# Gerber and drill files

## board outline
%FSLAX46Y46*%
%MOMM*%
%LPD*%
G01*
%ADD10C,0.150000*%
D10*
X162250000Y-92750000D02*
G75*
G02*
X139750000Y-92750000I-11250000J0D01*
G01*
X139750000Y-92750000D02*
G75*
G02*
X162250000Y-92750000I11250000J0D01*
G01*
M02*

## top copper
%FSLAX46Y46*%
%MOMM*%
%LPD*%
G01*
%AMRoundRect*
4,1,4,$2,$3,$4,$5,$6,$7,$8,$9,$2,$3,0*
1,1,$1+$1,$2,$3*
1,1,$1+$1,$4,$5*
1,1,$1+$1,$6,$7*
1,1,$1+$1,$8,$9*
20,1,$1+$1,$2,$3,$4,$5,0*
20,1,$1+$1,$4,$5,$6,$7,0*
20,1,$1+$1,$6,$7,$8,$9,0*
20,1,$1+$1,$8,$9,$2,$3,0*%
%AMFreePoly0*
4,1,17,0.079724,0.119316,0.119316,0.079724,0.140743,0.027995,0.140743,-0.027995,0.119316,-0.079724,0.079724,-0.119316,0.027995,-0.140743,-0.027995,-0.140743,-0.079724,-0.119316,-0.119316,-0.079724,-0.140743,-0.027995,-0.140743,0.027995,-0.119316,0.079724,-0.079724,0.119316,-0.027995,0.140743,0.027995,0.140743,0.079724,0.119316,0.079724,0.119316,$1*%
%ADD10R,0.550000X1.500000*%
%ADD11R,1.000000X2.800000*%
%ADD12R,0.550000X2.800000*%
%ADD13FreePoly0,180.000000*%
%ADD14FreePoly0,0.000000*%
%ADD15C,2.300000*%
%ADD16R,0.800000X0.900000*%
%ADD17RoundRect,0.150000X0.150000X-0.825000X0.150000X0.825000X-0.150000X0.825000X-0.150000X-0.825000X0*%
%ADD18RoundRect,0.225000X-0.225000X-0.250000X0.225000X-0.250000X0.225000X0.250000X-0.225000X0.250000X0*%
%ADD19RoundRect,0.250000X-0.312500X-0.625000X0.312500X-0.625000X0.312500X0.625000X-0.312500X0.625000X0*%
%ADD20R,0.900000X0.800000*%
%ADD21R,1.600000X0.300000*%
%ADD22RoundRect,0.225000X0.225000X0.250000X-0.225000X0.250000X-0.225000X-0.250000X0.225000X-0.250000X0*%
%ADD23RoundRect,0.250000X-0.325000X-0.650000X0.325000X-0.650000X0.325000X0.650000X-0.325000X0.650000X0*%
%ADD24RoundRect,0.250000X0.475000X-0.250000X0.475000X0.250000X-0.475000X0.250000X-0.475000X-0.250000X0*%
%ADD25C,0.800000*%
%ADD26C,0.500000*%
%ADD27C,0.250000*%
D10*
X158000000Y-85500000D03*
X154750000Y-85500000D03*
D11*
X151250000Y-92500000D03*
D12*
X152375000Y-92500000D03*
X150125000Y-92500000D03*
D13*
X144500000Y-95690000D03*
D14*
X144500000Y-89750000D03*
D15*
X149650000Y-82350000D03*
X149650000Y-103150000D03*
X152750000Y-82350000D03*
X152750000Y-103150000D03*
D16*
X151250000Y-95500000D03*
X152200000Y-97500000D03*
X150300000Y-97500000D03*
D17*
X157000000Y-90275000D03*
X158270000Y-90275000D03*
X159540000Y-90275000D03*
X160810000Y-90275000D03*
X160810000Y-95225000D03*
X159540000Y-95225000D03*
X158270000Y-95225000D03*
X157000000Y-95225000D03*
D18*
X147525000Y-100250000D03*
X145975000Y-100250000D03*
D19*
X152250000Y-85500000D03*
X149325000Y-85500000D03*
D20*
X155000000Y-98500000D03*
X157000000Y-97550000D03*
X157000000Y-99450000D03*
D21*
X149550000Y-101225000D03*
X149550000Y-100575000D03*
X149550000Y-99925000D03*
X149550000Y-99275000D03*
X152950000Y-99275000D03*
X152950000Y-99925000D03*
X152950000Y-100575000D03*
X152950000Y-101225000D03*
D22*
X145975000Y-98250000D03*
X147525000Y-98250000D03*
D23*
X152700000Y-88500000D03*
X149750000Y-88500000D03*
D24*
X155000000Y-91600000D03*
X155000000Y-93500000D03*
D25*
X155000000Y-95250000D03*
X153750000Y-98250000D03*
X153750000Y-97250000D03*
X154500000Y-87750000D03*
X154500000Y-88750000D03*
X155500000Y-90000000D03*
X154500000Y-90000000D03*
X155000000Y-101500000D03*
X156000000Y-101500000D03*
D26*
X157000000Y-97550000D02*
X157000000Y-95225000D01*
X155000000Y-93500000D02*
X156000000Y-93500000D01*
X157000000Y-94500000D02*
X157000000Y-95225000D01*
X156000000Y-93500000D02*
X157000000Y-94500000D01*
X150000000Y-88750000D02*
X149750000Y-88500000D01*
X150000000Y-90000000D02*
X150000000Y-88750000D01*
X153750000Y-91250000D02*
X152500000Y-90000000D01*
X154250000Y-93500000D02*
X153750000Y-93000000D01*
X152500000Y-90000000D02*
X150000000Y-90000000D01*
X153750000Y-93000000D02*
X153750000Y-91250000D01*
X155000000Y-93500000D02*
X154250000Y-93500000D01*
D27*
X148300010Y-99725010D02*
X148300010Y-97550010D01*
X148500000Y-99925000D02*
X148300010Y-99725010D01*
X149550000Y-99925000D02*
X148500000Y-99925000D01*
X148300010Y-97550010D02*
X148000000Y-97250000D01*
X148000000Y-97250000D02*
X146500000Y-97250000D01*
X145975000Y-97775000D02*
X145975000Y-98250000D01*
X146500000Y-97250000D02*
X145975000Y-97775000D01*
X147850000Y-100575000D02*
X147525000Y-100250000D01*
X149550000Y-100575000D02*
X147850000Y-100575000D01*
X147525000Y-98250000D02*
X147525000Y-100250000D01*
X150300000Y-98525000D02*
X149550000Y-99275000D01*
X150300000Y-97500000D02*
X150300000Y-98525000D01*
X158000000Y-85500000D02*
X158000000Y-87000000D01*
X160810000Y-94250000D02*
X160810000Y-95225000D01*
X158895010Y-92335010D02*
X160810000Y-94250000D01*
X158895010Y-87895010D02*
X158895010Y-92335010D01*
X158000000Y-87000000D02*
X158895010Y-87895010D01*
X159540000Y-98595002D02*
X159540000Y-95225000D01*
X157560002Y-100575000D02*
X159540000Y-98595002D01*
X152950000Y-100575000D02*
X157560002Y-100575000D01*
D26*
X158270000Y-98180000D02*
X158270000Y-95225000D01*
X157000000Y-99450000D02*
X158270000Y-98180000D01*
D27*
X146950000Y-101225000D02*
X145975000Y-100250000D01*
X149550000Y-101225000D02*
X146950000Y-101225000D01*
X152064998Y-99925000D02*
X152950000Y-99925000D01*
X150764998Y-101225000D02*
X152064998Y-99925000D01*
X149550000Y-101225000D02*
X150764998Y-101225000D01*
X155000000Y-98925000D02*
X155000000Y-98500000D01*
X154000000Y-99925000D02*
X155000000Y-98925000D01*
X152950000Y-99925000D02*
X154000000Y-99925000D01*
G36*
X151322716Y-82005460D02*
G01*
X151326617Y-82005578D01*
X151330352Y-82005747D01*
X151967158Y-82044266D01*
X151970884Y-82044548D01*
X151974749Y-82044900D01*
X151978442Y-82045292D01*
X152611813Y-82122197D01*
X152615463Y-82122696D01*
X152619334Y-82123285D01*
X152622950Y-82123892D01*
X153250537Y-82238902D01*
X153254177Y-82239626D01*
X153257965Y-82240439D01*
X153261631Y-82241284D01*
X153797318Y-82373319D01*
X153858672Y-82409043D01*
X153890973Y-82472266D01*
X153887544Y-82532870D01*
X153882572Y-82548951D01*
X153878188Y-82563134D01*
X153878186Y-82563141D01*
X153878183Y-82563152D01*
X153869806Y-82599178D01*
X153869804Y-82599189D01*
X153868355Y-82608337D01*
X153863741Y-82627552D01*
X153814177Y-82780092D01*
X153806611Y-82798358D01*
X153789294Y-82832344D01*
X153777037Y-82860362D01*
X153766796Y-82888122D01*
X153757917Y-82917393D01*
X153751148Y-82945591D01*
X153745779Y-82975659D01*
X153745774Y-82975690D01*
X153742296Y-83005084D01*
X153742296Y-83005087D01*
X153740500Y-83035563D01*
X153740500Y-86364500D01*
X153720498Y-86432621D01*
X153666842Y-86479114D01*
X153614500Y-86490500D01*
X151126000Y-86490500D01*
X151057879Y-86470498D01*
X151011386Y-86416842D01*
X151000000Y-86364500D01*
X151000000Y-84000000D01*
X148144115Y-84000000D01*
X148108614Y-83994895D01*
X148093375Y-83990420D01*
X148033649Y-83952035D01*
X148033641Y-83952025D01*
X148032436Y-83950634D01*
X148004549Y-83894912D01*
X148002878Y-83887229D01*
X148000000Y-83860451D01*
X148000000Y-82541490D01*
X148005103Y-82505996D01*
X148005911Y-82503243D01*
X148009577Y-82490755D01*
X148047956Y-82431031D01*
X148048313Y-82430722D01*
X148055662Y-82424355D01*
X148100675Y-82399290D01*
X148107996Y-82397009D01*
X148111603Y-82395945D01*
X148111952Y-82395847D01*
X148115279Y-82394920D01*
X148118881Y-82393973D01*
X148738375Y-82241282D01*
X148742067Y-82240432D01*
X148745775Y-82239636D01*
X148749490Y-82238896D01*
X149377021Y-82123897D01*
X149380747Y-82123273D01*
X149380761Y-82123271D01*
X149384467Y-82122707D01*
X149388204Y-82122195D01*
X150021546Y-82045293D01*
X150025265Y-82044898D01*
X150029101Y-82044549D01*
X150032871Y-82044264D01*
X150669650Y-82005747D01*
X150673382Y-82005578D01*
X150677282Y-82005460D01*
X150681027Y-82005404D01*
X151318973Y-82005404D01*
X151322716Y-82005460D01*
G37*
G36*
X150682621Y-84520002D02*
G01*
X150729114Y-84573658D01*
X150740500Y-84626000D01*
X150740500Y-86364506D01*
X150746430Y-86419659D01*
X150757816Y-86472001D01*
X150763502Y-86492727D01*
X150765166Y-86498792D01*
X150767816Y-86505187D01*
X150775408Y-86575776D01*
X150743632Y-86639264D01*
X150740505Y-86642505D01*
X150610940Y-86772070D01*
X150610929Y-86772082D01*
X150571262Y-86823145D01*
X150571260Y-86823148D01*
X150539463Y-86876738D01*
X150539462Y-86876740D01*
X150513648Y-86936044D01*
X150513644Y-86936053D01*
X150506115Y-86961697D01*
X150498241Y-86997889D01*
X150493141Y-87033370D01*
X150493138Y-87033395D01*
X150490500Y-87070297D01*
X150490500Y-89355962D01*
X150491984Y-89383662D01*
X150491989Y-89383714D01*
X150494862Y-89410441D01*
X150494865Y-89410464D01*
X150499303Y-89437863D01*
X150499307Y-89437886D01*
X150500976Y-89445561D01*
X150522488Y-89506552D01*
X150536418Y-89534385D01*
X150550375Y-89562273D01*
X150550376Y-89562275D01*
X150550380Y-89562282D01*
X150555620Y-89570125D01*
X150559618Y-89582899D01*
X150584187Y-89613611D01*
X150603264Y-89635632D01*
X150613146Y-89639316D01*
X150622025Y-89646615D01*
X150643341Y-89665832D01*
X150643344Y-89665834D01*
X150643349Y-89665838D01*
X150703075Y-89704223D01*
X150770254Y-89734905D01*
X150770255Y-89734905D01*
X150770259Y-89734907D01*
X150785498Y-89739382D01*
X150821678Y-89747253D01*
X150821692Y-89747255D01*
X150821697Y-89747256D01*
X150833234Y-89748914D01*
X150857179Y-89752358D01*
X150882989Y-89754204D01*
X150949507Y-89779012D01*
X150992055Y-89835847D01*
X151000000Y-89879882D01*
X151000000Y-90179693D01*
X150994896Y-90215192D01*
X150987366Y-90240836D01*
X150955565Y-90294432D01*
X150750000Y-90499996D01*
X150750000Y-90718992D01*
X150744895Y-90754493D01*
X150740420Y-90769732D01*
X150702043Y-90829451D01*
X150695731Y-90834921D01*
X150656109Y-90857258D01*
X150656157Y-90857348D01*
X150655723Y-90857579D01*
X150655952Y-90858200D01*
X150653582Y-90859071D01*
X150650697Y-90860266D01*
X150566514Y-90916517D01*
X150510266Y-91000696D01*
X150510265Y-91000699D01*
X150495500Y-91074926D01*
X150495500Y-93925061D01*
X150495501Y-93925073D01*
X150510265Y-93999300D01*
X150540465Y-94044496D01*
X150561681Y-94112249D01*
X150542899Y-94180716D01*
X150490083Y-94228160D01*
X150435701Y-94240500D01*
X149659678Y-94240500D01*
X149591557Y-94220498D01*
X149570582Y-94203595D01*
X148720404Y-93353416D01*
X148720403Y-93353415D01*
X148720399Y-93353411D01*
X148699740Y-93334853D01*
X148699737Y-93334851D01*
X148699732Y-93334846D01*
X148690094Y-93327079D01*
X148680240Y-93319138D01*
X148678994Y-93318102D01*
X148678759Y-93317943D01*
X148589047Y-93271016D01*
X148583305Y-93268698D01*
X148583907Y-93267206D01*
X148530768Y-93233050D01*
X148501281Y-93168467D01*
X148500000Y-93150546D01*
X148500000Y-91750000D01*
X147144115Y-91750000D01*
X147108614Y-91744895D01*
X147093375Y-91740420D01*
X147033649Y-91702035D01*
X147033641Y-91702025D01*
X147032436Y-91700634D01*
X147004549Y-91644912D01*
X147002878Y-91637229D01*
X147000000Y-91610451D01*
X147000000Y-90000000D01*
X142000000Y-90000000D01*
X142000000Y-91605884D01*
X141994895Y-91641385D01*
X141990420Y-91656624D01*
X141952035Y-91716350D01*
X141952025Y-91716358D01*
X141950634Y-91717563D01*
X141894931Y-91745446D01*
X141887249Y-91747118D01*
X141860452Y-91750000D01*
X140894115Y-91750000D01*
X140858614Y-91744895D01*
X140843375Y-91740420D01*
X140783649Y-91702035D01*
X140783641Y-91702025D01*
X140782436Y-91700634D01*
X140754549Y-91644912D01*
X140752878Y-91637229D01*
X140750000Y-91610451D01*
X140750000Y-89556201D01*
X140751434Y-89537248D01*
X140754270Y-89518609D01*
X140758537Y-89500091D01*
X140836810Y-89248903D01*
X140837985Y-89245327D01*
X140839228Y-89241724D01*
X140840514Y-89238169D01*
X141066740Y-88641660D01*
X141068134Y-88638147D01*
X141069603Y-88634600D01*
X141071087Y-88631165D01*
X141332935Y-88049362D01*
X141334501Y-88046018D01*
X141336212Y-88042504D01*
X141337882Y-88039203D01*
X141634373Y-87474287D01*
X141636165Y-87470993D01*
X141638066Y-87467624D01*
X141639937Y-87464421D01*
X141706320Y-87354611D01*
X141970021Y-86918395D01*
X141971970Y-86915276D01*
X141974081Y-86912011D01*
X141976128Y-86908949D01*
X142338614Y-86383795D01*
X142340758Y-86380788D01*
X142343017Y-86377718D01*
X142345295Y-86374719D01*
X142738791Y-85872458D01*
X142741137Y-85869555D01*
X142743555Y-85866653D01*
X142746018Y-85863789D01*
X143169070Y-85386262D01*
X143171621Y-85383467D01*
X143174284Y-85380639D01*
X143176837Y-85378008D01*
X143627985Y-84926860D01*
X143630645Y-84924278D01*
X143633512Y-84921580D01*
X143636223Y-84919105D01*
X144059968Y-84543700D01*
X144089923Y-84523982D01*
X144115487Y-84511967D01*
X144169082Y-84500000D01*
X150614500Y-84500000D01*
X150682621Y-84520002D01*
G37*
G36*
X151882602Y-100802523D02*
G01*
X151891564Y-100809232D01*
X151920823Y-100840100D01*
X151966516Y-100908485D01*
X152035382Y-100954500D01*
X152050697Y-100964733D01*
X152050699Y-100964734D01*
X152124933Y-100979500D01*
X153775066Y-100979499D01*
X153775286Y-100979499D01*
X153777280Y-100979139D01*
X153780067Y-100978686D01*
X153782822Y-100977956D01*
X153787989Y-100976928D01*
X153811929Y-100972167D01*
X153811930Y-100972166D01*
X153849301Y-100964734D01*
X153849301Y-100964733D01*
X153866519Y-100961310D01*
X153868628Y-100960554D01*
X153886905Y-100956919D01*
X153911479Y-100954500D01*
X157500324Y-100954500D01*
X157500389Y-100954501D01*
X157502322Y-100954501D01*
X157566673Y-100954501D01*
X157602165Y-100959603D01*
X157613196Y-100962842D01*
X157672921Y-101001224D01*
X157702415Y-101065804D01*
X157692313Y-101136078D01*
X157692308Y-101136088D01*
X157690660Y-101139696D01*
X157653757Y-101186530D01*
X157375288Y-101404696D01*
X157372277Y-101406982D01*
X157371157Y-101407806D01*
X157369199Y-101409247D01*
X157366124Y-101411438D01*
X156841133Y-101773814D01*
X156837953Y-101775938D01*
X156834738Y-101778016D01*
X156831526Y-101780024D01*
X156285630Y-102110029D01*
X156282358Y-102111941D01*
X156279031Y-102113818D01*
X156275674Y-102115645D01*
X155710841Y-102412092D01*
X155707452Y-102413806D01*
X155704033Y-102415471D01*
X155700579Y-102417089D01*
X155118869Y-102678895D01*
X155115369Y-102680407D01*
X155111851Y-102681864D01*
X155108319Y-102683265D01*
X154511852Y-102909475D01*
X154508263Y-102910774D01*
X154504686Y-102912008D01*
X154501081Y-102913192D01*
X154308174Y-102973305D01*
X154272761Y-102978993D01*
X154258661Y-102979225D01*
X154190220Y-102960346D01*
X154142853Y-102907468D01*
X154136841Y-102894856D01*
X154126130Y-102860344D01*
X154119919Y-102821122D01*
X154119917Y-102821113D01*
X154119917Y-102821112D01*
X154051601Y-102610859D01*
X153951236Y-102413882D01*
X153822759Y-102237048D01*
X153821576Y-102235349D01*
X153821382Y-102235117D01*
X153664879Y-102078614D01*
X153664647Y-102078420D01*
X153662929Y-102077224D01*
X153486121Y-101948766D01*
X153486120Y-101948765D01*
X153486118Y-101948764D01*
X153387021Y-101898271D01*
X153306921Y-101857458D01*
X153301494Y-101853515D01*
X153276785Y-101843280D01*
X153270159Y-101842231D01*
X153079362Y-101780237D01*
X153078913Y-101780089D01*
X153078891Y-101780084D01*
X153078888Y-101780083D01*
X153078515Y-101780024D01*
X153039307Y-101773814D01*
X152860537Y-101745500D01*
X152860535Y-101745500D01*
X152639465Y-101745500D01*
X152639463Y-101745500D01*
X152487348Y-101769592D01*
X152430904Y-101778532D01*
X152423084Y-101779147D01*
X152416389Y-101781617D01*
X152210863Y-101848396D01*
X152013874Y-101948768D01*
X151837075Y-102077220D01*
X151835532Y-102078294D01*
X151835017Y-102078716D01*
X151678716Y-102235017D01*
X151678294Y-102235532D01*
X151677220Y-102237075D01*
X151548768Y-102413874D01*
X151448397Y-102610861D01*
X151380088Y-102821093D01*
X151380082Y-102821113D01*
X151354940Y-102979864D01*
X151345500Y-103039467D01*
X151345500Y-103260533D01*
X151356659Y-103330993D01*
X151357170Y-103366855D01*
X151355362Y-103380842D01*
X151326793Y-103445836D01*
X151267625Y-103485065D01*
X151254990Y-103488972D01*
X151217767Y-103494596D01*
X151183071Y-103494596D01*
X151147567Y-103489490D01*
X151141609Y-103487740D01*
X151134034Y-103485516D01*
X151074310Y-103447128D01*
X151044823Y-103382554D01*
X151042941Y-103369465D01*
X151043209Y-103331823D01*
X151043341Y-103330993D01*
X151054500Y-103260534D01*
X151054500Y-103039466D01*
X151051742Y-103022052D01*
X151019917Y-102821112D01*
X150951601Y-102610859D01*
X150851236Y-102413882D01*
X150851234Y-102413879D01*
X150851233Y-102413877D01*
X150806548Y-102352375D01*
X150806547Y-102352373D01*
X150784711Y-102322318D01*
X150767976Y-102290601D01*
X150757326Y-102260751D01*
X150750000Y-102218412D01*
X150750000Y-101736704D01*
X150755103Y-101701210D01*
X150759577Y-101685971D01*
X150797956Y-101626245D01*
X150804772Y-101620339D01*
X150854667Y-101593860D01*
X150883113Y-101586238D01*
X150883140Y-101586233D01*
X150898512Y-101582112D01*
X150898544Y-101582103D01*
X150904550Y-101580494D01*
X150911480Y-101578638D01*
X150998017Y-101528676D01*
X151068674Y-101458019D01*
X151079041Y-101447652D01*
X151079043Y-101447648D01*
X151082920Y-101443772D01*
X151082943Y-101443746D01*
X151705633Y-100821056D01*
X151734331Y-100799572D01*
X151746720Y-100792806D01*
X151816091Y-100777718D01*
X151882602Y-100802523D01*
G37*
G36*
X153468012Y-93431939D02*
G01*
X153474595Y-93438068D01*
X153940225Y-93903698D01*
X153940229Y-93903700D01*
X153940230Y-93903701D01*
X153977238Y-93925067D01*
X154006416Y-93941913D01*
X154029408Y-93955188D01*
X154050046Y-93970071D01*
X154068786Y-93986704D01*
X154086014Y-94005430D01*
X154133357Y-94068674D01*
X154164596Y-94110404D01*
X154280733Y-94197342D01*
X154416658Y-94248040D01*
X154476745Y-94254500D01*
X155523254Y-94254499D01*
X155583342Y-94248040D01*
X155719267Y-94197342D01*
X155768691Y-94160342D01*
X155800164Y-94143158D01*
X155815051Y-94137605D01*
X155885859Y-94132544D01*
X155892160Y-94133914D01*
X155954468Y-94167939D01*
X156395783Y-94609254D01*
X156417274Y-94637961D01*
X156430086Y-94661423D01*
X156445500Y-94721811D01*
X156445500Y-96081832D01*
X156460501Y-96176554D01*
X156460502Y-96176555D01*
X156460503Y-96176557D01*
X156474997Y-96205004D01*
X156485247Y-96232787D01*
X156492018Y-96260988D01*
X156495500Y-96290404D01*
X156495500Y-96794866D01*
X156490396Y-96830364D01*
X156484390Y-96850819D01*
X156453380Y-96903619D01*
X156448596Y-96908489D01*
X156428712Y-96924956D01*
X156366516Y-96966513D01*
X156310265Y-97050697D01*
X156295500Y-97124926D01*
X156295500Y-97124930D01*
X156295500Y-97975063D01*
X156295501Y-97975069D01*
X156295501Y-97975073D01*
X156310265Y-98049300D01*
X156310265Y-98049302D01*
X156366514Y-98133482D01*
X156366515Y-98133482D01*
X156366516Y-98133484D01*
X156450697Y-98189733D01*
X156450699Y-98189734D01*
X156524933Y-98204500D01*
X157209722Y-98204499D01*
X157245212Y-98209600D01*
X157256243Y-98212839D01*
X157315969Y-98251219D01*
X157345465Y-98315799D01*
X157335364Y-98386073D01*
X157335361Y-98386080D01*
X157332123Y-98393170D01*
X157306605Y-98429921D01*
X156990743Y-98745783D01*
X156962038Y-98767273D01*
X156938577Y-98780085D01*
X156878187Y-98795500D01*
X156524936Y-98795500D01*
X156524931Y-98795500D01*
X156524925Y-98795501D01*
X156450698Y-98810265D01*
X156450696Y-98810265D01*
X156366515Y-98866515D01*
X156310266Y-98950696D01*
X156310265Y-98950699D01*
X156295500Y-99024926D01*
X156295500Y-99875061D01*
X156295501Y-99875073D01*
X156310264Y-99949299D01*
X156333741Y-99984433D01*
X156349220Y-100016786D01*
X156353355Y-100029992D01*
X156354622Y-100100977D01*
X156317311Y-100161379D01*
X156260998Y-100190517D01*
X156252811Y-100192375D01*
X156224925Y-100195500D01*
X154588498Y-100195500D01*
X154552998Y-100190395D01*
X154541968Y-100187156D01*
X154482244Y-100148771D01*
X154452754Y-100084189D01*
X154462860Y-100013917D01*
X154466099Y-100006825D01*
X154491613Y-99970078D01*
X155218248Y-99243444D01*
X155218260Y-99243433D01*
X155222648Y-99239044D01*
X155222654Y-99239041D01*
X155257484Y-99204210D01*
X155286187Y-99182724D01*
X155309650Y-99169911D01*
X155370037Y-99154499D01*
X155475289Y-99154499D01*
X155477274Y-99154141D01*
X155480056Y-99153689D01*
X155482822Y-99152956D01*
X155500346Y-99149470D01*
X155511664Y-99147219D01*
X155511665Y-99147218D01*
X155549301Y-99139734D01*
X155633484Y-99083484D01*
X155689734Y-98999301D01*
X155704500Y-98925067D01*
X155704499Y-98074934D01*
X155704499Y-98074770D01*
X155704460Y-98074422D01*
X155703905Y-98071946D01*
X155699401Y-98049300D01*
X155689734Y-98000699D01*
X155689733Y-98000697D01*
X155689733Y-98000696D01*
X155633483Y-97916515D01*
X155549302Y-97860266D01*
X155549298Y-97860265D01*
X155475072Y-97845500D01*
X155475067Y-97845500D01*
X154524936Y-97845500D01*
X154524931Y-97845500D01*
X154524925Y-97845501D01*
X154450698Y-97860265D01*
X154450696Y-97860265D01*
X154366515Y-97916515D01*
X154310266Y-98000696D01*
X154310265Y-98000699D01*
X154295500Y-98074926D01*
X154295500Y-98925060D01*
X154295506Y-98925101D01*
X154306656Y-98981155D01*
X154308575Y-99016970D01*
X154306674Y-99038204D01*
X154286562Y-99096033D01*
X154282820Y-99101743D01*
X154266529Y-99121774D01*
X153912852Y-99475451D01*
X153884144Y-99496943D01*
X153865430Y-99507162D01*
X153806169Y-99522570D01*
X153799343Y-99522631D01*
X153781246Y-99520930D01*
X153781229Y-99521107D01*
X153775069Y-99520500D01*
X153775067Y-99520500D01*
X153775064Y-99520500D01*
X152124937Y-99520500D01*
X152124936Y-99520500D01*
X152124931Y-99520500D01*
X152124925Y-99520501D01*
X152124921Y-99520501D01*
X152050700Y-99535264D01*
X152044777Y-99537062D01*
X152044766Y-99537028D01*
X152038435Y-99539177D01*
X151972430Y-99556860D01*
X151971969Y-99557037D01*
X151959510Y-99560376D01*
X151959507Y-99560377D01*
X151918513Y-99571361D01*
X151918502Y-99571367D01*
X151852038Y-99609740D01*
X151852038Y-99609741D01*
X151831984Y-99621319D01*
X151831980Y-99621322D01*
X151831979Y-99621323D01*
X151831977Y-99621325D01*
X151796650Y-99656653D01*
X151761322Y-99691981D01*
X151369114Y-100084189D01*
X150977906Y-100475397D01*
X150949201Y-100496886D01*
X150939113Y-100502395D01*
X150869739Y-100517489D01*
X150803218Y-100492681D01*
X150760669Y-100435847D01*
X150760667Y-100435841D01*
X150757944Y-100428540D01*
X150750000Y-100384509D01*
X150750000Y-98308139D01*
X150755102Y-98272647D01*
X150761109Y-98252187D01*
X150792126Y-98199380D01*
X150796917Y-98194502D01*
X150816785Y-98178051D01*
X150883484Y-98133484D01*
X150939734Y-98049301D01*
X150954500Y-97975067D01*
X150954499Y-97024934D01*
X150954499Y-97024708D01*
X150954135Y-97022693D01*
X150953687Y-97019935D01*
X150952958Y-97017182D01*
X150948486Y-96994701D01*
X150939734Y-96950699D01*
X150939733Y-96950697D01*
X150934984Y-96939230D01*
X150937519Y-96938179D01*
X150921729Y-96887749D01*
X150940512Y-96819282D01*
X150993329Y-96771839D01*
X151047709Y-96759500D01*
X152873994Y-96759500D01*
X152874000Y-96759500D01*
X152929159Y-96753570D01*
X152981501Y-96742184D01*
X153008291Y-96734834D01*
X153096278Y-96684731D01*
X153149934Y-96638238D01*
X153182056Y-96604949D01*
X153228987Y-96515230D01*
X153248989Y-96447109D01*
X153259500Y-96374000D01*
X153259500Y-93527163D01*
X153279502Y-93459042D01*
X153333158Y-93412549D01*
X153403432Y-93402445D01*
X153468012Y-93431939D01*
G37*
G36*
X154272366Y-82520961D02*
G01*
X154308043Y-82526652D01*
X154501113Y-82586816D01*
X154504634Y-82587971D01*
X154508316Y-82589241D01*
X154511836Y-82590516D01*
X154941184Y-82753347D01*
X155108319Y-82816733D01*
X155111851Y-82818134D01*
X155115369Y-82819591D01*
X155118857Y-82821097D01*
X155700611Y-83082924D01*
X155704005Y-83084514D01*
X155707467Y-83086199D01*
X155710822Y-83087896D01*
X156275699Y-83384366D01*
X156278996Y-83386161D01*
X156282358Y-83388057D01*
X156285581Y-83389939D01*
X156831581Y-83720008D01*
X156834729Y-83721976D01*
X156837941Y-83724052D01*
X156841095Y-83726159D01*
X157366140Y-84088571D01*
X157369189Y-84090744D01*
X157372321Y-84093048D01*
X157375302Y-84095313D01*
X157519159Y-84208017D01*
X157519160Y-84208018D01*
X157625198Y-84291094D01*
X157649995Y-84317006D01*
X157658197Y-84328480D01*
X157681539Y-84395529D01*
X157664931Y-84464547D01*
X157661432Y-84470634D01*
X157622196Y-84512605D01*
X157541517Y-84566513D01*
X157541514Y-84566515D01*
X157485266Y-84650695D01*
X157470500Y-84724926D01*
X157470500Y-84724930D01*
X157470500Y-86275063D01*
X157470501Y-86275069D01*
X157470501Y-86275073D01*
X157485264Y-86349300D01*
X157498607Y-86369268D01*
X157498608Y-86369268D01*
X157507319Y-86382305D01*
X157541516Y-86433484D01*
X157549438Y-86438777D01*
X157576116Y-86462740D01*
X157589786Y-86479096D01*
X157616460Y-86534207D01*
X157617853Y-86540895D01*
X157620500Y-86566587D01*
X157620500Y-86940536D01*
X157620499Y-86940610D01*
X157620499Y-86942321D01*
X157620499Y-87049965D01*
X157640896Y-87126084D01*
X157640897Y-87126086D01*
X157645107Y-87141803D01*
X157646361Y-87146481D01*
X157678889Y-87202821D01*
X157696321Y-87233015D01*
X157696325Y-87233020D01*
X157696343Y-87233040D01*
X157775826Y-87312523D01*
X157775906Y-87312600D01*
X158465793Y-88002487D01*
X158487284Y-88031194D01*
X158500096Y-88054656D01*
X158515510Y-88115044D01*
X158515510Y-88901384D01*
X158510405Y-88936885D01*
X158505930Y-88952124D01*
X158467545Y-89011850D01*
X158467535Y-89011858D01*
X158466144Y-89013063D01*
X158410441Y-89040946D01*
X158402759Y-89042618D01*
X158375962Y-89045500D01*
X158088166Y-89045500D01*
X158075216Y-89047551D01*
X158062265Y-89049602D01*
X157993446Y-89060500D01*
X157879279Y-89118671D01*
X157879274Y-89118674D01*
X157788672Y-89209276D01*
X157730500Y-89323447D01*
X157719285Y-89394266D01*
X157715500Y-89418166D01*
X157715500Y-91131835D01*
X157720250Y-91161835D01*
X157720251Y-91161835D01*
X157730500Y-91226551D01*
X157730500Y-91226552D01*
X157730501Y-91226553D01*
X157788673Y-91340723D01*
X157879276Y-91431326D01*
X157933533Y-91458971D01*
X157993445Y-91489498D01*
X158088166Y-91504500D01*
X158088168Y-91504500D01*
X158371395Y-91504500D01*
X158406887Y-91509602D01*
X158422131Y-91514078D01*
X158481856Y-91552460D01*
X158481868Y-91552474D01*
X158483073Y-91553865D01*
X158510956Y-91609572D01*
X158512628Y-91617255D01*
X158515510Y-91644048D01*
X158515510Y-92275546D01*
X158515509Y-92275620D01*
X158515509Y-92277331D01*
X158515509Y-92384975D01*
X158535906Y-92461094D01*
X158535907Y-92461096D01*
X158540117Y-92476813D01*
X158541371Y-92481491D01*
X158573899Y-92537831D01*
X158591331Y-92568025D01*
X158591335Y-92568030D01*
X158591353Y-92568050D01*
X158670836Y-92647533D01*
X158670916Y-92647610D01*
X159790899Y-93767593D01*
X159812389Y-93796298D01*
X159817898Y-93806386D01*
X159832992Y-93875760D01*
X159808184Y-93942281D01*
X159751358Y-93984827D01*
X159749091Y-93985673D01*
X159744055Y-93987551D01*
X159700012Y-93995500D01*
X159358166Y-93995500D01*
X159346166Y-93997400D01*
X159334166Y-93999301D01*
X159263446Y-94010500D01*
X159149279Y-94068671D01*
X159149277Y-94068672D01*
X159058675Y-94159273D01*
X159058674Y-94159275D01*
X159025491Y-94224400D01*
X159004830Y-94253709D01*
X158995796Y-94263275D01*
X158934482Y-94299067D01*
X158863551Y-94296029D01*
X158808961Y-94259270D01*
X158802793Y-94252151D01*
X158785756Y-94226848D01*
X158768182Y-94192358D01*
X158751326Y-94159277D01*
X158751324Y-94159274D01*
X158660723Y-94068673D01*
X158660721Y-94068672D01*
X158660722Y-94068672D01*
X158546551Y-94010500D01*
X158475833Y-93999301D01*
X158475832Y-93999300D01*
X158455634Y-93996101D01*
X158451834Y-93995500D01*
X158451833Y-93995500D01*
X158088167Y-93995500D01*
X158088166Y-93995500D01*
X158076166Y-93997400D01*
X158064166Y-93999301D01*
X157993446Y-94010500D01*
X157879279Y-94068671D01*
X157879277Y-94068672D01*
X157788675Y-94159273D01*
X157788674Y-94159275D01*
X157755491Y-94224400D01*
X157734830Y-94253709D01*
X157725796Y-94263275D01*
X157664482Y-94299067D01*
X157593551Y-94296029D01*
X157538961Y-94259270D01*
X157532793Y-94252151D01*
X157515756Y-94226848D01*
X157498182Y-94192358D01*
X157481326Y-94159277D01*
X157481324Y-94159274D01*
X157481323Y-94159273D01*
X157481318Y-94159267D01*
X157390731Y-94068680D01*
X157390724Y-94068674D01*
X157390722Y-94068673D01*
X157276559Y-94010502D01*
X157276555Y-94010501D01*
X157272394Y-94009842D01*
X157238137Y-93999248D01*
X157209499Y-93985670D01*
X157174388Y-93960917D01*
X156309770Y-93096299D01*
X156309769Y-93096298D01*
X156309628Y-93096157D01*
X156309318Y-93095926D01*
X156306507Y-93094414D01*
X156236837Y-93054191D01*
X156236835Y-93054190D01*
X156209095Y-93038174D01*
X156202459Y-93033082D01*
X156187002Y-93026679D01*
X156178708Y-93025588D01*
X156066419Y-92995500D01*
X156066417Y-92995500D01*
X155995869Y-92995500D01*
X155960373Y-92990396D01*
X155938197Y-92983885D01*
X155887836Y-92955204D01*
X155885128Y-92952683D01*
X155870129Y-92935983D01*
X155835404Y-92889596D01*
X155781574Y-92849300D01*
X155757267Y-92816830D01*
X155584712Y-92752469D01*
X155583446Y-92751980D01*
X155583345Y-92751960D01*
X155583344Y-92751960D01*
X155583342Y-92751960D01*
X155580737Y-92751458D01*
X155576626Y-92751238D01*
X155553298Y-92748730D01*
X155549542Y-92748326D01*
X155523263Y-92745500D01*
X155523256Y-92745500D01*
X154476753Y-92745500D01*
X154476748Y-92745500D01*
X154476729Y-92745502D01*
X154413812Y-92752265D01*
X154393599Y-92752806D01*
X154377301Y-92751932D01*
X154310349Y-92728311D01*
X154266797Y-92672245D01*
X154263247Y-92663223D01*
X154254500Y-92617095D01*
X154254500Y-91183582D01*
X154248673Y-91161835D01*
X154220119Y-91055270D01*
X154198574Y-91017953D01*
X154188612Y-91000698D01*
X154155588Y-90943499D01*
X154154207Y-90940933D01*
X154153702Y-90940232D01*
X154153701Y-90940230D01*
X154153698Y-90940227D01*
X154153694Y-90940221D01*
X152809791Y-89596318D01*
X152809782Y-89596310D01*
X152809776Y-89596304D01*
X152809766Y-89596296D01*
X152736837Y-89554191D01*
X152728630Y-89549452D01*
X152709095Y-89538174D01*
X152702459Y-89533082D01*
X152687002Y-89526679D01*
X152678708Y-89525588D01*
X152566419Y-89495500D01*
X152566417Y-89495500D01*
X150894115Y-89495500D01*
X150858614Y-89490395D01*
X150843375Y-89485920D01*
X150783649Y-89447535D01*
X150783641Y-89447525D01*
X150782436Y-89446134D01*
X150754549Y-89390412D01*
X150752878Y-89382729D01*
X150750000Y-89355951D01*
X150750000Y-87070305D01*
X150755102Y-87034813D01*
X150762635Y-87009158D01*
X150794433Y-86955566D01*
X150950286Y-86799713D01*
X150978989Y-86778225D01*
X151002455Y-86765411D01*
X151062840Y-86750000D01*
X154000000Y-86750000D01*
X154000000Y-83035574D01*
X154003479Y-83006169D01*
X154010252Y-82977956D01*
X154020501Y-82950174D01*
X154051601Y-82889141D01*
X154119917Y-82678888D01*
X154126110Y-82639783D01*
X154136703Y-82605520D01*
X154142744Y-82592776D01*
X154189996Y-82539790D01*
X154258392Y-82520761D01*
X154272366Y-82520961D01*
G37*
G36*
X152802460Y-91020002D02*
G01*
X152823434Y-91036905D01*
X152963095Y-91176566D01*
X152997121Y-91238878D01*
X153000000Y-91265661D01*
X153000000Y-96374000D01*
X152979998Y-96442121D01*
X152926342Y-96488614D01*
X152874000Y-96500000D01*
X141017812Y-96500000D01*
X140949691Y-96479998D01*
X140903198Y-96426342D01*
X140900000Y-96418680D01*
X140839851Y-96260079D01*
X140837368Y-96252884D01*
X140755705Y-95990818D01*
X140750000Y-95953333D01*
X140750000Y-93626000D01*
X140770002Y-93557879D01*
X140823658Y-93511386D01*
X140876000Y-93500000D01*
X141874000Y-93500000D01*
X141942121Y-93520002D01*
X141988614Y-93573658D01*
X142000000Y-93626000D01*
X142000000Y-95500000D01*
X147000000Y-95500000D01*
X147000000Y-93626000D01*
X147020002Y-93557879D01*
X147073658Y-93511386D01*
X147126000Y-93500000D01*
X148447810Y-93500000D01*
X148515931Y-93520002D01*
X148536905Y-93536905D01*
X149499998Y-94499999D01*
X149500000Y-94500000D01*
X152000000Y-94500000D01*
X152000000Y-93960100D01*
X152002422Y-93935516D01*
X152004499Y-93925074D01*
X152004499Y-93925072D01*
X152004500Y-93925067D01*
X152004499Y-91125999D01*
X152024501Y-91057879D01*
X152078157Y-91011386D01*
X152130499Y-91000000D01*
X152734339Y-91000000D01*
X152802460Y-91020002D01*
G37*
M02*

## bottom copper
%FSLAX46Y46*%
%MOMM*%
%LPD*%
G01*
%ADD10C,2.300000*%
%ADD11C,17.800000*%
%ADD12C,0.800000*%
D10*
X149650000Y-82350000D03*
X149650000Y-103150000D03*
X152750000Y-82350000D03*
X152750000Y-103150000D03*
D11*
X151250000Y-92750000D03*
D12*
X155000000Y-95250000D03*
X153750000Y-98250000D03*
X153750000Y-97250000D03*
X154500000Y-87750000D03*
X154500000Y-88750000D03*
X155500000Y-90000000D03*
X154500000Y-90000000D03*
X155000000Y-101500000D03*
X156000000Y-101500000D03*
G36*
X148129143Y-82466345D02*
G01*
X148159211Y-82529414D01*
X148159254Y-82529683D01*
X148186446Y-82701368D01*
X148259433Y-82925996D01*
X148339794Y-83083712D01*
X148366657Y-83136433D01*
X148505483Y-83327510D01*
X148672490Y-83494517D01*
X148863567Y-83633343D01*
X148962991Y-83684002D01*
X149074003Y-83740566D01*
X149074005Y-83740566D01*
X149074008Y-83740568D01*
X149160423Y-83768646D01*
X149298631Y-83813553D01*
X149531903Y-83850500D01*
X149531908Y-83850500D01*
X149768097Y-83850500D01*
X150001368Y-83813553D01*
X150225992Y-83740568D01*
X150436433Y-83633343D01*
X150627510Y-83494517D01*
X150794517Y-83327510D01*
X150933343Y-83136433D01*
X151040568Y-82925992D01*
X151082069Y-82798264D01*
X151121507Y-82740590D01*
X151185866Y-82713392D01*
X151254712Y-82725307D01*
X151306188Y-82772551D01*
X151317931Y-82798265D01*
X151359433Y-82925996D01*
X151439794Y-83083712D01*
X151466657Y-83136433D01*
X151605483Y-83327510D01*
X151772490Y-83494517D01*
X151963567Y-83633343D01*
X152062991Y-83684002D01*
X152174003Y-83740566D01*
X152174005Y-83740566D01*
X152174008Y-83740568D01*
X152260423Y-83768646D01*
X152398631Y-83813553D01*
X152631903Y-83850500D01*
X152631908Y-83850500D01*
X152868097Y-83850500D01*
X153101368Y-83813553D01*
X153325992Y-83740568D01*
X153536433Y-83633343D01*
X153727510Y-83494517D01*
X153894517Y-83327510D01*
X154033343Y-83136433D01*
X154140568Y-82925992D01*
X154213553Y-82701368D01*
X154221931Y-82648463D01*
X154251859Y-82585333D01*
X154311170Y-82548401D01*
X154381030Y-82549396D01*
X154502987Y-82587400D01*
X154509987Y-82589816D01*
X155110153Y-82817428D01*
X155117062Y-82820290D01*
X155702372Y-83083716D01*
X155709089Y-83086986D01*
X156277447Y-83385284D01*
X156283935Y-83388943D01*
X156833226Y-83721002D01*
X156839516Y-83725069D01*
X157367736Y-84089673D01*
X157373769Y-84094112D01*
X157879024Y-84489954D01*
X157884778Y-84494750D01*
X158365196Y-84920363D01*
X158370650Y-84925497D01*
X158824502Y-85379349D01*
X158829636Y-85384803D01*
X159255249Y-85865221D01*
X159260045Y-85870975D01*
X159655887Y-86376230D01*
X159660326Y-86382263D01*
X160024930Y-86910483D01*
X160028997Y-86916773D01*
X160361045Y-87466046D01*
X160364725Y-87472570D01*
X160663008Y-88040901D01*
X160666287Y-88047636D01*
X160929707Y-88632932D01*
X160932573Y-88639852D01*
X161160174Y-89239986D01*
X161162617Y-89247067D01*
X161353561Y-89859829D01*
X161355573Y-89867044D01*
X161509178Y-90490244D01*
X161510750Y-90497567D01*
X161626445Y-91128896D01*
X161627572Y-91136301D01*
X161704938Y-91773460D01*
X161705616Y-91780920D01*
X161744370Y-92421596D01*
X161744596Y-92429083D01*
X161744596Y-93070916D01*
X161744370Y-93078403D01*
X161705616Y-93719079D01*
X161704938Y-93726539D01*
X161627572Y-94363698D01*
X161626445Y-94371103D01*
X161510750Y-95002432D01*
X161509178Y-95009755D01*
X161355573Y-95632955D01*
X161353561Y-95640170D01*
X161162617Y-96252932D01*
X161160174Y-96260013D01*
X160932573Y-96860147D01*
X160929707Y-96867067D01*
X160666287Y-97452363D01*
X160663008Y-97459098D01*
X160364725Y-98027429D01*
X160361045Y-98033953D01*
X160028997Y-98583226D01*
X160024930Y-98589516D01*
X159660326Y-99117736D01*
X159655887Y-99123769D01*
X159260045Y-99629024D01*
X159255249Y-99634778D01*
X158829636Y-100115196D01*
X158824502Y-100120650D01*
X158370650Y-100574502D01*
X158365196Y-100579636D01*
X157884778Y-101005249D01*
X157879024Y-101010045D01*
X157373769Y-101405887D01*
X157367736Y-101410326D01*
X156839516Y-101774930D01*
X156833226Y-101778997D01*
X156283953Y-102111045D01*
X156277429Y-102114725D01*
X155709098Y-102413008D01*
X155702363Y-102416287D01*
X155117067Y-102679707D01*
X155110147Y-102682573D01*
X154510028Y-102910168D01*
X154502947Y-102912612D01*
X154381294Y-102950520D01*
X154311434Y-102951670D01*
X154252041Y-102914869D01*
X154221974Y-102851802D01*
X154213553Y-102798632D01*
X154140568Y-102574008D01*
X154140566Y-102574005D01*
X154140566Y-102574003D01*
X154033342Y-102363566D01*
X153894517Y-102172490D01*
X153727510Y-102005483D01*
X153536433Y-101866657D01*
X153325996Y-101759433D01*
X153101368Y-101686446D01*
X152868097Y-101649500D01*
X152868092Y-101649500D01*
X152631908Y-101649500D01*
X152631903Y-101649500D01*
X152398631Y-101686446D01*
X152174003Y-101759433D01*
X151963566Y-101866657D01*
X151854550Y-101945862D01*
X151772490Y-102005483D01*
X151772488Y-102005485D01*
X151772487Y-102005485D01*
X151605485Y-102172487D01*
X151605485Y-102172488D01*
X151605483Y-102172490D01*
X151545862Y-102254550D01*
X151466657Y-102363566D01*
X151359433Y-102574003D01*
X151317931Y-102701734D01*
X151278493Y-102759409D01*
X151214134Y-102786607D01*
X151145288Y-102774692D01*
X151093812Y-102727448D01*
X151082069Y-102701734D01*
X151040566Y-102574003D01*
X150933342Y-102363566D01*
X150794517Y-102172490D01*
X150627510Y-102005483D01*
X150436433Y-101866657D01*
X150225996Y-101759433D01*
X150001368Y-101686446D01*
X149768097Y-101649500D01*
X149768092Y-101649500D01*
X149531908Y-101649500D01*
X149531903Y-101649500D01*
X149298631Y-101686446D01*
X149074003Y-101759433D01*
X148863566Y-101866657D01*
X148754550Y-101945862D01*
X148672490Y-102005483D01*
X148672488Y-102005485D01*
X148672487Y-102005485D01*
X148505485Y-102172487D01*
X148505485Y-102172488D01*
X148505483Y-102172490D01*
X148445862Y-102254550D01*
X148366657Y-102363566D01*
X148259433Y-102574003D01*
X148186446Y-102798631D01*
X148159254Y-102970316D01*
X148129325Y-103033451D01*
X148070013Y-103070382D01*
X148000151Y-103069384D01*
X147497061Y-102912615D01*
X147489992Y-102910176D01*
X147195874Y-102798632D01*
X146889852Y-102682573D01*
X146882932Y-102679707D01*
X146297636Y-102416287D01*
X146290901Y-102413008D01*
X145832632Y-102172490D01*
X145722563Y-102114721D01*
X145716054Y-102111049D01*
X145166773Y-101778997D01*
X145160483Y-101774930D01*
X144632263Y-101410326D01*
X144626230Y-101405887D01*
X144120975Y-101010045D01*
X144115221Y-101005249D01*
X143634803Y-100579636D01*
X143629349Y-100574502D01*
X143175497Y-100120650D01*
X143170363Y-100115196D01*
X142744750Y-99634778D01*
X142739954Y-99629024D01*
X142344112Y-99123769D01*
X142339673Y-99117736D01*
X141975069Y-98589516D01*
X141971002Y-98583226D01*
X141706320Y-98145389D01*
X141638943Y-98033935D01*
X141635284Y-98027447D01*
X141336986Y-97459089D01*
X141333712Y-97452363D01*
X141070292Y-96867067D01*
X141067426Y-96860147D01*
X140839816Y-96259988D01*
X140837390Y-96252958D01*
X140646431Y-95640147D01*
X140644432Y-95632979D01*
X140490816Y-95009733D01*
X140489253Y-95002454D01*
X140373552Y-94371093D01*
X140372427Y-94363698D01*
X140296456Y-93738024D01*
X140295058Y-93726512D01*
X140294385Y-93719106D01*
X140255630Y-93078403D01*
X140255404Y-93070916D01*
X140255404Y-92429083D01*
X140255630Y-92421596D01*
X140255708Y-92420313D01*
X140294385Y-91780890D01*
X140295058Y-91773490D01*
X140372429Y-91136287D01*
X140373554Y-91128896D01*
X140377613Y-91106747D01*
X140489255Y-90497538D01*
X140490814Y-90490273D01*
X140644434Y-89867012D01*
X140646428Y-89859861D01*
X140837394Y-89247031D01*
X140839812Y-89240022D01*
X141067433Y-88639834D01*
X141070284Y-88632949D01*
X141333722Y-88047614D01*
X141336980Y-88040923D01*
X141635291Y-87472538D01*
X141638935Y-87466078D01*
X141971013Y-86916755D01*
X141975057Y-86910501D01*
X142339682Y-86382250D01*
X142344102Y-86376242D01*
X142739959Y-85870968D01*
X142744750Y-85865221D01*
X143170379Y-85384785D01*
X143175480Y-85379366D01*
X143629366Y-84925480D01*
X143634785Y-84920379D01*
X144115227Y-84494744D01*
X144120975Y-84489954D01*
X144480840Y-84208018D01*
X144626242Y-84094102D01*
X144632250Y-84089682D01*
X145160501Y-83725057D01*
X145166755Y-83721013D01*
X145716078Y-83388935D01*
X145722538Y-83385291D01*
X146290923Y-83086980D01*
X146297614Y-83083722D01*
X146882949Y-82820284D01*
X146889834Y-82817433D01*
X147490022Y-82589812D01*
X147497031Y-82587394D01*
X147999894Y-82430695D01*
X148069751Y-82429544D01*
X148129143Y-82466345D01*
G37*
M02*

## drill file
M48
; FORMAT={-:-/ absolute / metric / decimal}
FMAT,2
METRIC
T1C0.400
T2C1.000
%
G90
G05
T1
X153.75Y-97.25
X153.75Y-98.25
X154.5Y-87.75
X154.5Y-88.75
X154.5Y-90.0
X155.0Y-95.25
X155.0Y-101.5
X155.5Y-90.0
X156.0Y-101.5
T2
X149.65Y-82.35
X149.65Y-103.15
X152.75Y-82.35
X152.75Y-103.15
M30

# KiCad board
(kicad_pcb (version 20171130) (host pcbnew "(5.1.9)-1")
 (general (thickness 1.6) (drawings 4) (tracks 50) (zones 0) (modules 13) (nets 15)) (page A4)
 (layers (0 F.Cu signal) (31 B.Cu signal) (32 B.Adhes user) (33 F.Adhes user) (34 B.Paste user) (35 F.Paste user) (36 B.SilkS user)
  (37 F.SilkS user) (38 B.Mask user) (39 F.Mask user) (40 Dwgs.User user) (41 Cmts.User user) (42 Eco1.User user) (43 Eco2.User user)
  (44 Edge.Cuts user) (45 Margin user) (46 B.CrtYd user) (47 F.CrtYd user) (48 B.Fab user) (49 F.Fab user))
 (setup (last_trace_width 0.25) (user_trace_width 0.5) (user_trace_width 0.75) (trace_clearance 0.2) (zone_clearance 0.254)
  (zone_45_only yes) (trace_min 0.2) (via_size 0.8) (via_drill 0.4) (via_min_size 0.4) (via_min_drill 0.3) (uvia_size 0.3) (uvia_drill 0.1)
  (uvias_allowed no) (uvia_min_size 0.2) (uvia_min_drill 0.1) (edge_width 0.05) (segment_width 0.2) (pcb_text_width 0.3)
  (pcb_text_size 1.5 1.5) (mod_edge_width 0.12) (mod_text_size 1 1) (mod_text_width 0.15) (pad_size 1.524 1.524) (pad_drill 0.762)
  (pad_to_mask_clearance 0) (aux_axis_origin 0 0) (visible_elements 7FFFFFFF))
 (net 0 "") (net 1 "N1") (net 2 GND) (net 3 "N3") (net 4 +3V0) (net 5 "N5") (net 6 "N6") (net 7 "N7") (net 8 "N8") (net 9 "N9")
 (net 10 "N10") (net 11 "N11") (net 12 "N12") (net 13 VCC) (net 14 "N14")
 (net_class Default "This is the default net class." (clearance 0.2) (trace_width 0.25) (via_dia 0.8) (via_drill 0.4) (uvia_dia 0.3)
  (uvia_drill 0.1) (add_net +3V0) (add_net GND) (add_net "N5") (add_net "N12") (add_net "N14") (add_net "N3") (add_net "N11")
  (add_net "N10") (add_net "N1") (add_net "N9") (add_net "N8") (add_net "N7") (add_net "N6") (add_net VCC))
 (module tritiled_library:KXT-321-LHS (layer F.Cu) (at 154.75 85.5)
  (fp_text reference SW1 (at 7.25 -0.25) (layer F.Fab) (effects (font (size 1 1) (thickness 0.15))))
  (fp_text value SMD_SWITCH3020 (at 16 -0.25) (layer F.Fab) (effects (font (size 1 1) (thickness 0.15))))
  (pad 2 smd rect (at 3.25 0 90) (size 1.5 0.55) (layers F.Cu F.Paste F.Mask) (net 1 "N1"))
  (pad 1 smd rect (at 0 0 90) (size 1.5 0.55) (layers F.Cu F.Paste F.Mask) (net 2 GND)))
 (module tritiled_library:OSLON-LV (layer F.Cu) (at 151.25 92.5 270)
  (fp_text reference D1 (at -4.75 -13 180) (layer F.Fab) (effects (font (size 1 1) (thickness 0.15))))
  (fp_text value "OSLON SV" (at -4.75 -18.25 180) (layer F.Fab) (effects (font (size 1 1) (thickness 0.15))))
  (pad 3 smd rect (at 0 0 270) (size 2.8 1) (layers F.Cu F.Paste F.Mask) (solder_mask_margin 0.05) (solder_paste_margin -0.075))
  (pad 2 smd rect (at 0 -1.125 270) (size 2.8 0.55) (layers F.Cu F.Paste F.Mask) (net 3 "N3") (solder_mask_margin 0.05)
   (solder_paste_margin -0.075))
  (pad 1 smd rect (at 0 1.125 270) (size 2.8 0.55) (layers F.Cu F.Paste F.Mask) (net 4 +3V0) (solder_mask_margin 0.05)
   (solder_paste_margin -0.075)))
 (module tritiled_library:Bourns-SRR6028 (layer F.Cu) (at 144.5 92.72 270)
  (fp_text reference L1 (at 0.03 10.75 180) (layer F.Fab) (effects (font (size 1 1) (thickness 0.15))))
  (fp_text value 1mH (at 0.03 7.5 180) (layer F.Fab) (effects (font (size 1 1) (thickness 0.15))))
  (pad 2 smd custom (at 2.97 0 180) (size 0.287 0.287) (layers F.Cu F.Paste F.Mask) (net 3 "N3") (zone_connect 2)
   (options (clearance convexhull) (anchor circle)) (primitives))
  (pad 1 smd custom (at -2.97 0) (size 0.287 0.287) (layers F.Cu F.Paste F.Mask) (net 4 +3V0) (zone_connect 2)
   (options (clearance convexhull) (anchor circle)) (primitives)))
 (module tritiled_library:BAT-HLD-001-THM (layer B.Cu) (at 151.25 92.75 90)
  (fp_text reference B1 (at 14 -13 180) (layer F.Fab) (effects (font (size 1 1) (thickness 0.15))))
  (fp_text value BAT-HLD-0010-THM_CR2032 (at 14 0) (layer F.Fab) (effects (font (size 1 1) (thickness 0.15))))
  (pad 1 thru_hole circle (at 10.4 -1.6 90) (size 2.3 2.3) (drill 1) (layers *.Cu *.Mask) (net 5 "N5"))
  (pad 1 thru_hole circle (at -10.4 -1.6 90) (size 2.3 2.3) (drill 1) (layers *.Cu *.Mask) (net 5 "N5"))
  (pad 1 thru_hole circle (at 10.4 1.5 90) (size 2.3 2.3) (drill 1) (layers *.Cu *.Mask) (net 5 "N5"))
  (pad 1 thru_hole circle (at -10.4 1.5 90) (size 2.3 2.3) (drill 1) (layers *.Cu *.Mask) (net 5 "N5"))
  (pad 2 smd circle (at 0 0 90) (size 17.8 17.8) (layers B.Cu B.Paste B.Mask) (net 2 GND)))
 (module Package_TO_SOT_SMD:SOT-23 (layer F.Cu) (at 151.25 96.5 90)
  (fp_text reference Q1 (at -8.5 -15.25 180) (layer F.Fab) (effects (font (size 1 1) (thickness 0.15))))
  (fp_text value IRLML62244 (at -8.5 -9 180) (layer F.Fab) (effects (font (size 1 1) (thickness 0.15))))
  (pad 3 smd rect (at 1 0 90) (size 0.9 0.8) (layers F.Cu F.Paste F.Mask) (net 3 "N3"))
  (pad 2 smd rect (at -1 0.95 90) (size 0.9 0.8) (layers F.Cu F.Paste F.Mask) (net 2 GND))
  (pad 1 smd rect (at -1 -0.95 90) (size 0.9 0.8) (layers F.Cu F.Paste F.Mask) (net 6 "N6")))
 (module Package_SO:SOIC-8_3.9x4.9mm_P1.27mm (layer F.Cu) (at 158.905 92.75 90)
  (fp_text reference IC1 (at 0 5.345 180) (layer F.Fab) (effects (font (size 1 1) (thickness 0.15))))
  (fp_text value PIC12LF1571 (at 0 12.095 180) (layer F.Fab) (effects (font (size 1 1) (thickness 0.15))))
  (pad 8 smd roundrect (at 2.475 -1.905 90) (size 1.95 0.6) (layers F.Cu F.Paste F.Mask) (roundrect_rratio 0.25) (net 2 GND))
  (pad 7 smd roundrect (at 2.475 -0.635 90) (size 1.95 0.6) (layers F.Cu F.Paste F.Mask) (roundrect_rratio 0.25) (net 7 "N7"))
  (pad 6 smd roundrect (at 2.475 0.635 90) (size 1.95 0.6) (layers F.Cu F.Paste F.Mask) (roundrect_rratio 0.25) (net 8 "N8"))
  (pad 5 smd roundrect (at 2.475 1.905 90) (size 1.95 0.6) (layers F.Cu F.Paste F.Mask) (roundrect_rratio 0.25) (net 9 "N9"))
  (pad 4 smd roundrect (at -2.475 1.905 90) (size 1.95 0.6) (layers F.Cu F.Paste F.Mask) (roundrect_rratio 0.25) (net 1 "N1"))
  (pad 3 smd roundrect (at -2.475 0.635 90) (size 1.95 0.6) (layers F.Cu F.Paste F.Mask) (roundrect_rratio 0.25) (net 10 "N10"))
  (pad 2 smd roundrect (at -2.475 -0.635 90) (size 1.95 0.6) (layers F.Cu F.Paste F.Mask) (roundrect_rratio 0.25) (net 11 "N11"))
  (pad 1 smd roundrect (at -2.475 -1.905 90) (size 1.95 0.6) (layers F.Cu F.Paste F.Mask) (roundrect_rratio 0.25) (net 4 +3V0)))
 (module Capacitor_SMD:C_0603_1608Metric (layer F.Cu) (at 146.75 100.25)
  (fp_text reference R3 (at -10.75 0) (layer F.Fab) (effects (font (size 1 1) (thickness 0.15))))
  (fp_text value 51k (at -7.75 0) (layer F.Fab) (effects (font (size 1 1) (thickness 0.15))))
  (pad 2 smd roundrect (at 0.775 0) (size 0.9 0.95) (layers F.Cu F.Paste F.Mask) (roundrect_rratio 0.25) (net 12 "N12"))
  (pad 1 smd roundrect (at -0.775 0) (size 0.9 0.95) (layers F.Cu F.Paste F.Mask) (roundrect_rratio 0.25) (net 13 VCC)))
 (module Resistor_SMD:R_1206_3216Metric (layer F.Cu) (at 150.7875 85.5)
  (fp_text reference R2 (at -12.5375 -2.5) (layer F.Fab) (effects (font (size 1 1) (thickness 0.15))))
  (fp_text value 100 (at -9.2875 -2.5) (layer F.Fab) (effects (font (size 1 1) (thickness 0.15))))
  (pad 2 smd roundrect (at 1.4625 0) (size 1.125 1.75) (layers F.Cu F.Paste F.Mask) (roundrect_rratio 0.222222) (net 5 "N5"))
  (pad 1 smd roundrect (at -1.4625 0) (size 1.125 1.75) (layers F.Cu F.Paste F.Mask) (roundrect_rratio 0.222222) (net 4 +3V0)))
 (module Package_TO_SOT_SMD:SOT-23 (layer F.Cu) (at 156 98.5 180)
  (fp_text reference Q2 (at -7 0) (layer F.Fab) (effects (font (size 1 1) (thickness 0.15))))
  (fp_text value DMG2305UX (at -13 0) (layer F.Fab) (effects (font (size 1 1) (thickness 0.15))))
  (pad 3 smd rect (at 1 0 180) (size 0.9 0.8) (layers F.Cu F.Paste F.Mask) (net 13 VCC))
  (pad 2 smd rect (at -1 0.95 180) (size 0.9 0.8) (layers F.Cu F.Paste F.Mask) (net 4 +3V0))
  (pad 1 smd rect (at -1 -0.95 180) (size 0.9 0.8) (layers F.Cu F.Paste F.Mask) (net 11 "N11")))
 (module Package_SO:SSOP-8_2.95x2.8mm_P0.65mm (layer F.Cu) (at 151.25 100.25 180)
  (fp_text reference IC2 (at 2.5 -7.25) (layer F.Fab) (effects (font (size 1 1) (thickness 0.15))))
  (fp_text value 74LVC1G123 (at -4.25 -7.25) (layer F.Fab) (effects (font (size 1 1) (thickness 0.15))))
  (pad 8 smd rect (at 1.7 -0.975 90) (size 0.3 1.6) (layers F.Cu F.Paste F.Mask) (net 13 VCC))
  (pad 7 smd rect (at 1.7 -0.325 90) (size 0.3 1.6) (layers F.Cu F.Paste F.Mask) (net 12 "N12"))
  (pad 6 smd rect (at 1.7 0.325 90) (size 0.3 1.6) (layers F.Cu F.Paste F.Mask) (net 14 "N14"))
  (pad 5 smd rect (at 1.7 0.975 90) (size 0.3 1.6) (layers F.Cu F.Paste F.Mask) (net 6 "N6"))
  (pad 4 smd rect (at -1.7 0.975 90) (size 0.3 1.6) (layers F.Cu F.Paste F.Mask) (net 2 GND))
  (pad 3 smd rect (at -1.7 0.325 90) (size 0.3 1.6) (layers F.Cu F.Paste F.Mask) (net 13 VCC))
  (pad 2 smd rect (at -1.7 -0.325 90) (size 0.3 1.6) (layers F.Cu F.Paste F.Mask) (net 10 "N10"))
  (pad 1 smd rect (at -1.7 -0.975 90) (size 0.3 1.6) (layers F.Cu F.Paste F.Mask) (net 2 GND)))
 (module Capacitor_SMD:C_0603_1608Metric (layer F.Cu) (at 146.75 98.25 180)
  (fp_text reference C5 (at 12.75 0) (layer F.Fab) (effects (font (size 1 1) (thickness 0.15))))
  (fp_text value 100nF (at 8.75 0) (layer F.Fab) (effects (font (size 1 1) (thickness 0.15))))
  (pad 2 smd roundrect (at 0.775 0 180) (size 0.9 0.95) (layers F.Cu F.Paste F.Mask) (roundrect_rratio 0.25) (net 14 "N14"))
  (pad 1 smd roundrect (at -0.775 0 180) (size 0.9 0.95) (layers F.Cu F.Paste F.Mask) (roundrect_rratio 0.25) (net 12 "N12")))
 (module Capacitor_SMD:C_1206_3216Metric (layer F.Cu) (at 151.225 88.5)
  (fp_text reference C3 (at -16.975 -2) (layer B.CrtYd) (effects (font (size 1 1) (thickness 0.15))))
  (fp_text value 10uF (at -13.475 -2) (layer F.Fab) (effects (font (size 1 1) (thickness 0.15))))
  (pad 2 smd roundrect (at 1.475 0) (size 1.15 1.8) (layers F.Cu F.Paste F.Mask) (roundrect_rratio 0.217391) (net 2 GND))
  (pad 1 smd roundrect (at -1.475 0) (size 1.15 1.8) (layers F.Cu F.Paste F.Mask) (roundrect_rratio 0.217391) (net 4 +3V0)))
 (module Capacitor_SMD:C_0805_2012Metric (layer F.Cu) (at 155 92.55 90)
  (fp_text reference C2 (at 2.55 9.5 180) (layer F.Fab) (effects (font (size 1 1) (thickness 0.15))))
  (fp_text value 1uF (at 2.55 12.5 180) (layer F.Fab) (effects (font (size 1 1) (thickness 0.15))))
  (pad 2 smd roundrect (at 0.95 0 90) (size 1 1.45) (layers F.Cu F.Paste F.Mask) (roundrect_rratio 0.25) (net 2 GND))
  (pad 1 smd roundrect (at -0.95 0 90) (size 1 1.45) (layers F.Cu F.Paste F.Mask) (roundrect_rratio 0.25) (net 4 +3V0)))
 (gr_circle (center 151 92.75) (end 162.25 92.75) (layer Edge.Cuts) (width 0.15))
 (via (at 155 95.25) (size 0.8) (drill 0.4) (layers F.Cu B.Cu) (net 2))
 (via (at 153.75 98.25) (size 0.8) (drill 0.4) (layers F.Cu B.Cu) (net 2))
 (via (at 153.75 97.25) (size 0.8) (drill 0.4) (layers F.Cu B.Cu) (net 2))
 (via (at 154.5 87.75) (size 0.8) (drill 0.4) (layers F.Cu B.Cu) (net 2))
 (via (at 154.5 88.75) (size 0.8) (drill 0.4) (layers F.Cu B.Cu) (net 2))
 (via (at 155.5 90) (size 0.8) (drill 0.4) (layers F.Cu B.Cu) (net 2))
 (via (at 154.5 90) (size 0.8) (drill 0.4) (layers F.Cu B.Cu) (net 2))
 (via (at 155 101.5) (size 0.8) (drill 0.4) (layers F.Cu B.Cu) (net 2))
 (via (at 156 101.5) (size 0.8) (drill 0.4) (layers F.Cu B.Cu) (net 2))
 (segment (start 157 97.55) (end 157 95.225) (width 0.5) (layer F.Cu) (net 4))
 (segment (start 155 93.5) (end 156 93.5) (width 0.5) (layer F.Cu) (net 4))
 (segment (start 157 94.5) (end 157 95.225) (width 0.5) (layer F.Cu) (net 4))
 (segment (start 156 93.5) (end 157 94.5) (width 0.5) (layer F.Cu) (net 4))
 (segment (start 150 88.75) (end 149.75 88.5) (width 0.5) (layer F.Cu) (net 4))
 (segment (start 150 90) (end 150 88.75) (width 0.5) (layer F.Cu) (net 4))
 (segment (start 153.75 91.25) (end 152.5 90) (width 0.5) (layer F.Cu) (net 4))
 (segment (start 154.25 93.5) (end 153.75 93) (width 0.5) (layer F.Cu) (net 4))
 (segment (start 152.5 90) (end 150 90) (width 0.5) (layer F.Cu) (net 4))
 (segment (start 153.75 93) (end 153.75 91.25) (width 0.5) (layer F.Cu) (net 4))
 (segment (start 155 93.5) (end 154.25 93.5) (width 0.5) (layer F.Cu) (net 4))
 (segment (start 148.30001 99.72501) (end 148.30001 97.55001) (width 0.25) (layer F.Cu) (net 14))
 (segment (start 148.5 99.925) (end 148.30001 99.72501) (width 0.25) (layer F.Cu) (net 14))
 (segment (start 149.55 99.925) (end 148.5 99.925) (width 0.25) (layer F.Cu) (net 14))
 (segment (start 148.30001 97.55001) (end 148 97.25) (width 0.25) (layer F.Cu) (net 14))
 (segment (start 148 97.25) (end 146.5 97.25) (width 0.25) (layer F.Cu) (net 14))
 (segment (start 145.975 97.775) (end 145.975 98.25) (width 0.25) (layer F.Cu) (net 14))
 (segment (start 146.5 97.25) (end 145.975 97.775) (width 0.25) (layer F.Cu) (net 14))
 (segment (start 147.85 100.575) (end 147.525 100.25) (width 0.25) (layer F.Cu) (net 12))
 (segment (start 149.55 100.575) (end 147.85 100.575) (width 0.25) (layer F.Cu) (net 12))
 (segment (start 147.525 98.25) (end 147.525 100.25) (width 0.25) (layer F.Cu) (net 12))
 (segment (start 150.3 98.525) (end 149.55 99.275) (width 0.25) (layer F.Cu) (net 6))
 (segment (start 150.3 97.5) (end 150.3 98.525) (width 0.25) (layer F.Cu) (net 6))
 (segment (start 158 85.5) (end 158 87) (width 0.25) (layer F.Cu) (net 1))
 (segment (start 160.81 94.25) (end 160.81 95.225) (width 0.25) (layer F.Cu) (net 1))
 (segment (start 158.89501 92.33501) (end 160.81 94.25) (width 0.25) (layer F.Cu) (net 1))
 (segment (start 158.89501 87.89501) (end 158.89501 92.33501) (width 0.25) (layer F.Cu) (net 1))
 (segment (start 158 87) (end 158.89501 87.89501) (width 0.25) (layer F.Cu) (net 1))
 (segment (start 159.54 98.595002) (end 159.54 95.225) (width 0.25) (layer F.Cu) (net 10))
 (segment (start 157.560002 100.575) (end 159.54 98.595002) (width 0.25) (layer F.Cu) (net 10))
 (segment (start 152.95 100.575) (end 157.560002 100.575) (width 0.25) (layer F.Cu) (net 10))
 (segment (start 158.27 98.18) (end 158.27 95.225) (width 0.5) (layer F.Cu) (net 11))
 (segment (start 157 99.45) (end 158.27 98.18) (width 0.5) (layer F.Cu) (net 11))
 (segment (start 146.95 101.225) (end 145.975 100.25) (width 0.25) (layer F.Cu) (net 13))
 (segment (start 149.55 101.225) (end 146.95 101.225) (width 0.25) (layer F.Cu) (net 13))
 (segment (start 152.064998 99.925) (end 152.95 99.925) (width 0.25) (layer F.Cu) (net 13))
 (segment (start 150.764998 101.225) (end 152.064998 99.925) (width 0.25) (layer F.Cu) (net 13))
 (segment (start 149.55 101.225) (end 150.764998 101.225) (width 0.25) (layer F.Cu) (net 13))
 (segment (start 155 98.925) (end 155 98.5) (width 0.25) (layer F.Cu) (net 13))
 (segment (start 154 99.925) (end 155 98.925) (width 0.25) (layer F.Cu) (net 13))
 (segment (start 152.95 99.925) (end 154 99.925) (width 0.25) (layer F.Cu) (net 13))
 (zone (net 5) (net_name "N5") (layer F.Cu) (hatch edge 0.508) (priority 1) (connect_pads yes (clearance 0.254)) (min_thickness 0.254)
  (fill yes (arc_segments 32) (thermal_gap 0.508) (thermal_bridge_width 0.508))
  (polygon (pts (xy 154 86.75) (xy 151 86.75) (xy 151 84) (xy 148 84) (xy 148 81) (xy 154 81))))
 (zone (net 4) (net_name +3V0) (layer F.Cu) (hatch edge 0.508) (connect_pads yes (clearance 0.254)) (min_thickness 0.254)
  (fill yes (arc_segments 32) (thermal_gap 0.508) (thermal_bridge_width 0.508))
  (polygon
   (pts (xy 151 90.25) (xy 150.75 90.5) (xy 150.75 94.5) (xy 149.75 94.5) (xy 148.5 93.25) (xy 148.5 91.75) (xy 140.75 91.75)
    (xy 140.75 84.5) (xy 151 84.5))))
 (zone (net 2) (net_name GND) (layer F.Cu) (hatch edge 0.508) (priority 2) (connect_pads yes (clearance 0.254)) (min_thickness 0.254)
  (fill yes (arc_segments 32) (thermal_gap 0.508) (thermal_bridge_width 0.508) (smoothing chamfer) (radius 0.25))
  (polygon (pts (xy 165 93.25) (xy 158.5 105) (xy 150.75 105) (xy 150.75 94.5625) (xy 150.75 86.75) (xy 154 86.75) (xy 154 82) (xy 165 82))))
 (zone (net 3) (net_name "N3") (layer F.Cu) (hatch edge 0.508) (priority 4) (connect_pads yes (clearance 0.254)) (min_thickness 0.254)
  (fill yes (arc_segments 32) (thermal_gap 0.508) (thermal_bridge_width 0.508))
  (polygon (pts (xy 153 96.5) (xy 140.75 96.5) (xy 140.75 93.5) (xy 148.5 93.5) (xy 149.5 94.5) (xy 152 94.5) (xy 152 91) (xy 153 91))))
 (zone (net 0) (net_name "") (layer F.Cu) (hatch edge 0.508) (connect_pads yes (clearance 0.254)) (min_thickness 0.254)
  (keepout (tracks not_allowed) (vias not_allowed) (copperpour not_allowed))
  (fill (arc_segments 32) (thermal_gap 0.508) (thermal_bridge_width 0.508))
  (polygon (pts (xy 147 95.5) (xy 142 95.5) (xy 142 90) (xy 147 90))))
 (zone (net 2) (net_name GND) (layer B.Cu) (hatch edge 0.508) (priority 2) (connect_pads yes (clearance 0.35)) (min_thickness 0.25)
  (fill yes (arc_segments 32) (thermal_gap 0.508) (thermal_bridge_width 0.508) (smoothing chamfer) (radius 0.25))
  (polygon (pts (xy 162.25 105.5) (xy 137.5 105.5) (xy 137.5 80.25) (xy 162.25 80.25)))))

